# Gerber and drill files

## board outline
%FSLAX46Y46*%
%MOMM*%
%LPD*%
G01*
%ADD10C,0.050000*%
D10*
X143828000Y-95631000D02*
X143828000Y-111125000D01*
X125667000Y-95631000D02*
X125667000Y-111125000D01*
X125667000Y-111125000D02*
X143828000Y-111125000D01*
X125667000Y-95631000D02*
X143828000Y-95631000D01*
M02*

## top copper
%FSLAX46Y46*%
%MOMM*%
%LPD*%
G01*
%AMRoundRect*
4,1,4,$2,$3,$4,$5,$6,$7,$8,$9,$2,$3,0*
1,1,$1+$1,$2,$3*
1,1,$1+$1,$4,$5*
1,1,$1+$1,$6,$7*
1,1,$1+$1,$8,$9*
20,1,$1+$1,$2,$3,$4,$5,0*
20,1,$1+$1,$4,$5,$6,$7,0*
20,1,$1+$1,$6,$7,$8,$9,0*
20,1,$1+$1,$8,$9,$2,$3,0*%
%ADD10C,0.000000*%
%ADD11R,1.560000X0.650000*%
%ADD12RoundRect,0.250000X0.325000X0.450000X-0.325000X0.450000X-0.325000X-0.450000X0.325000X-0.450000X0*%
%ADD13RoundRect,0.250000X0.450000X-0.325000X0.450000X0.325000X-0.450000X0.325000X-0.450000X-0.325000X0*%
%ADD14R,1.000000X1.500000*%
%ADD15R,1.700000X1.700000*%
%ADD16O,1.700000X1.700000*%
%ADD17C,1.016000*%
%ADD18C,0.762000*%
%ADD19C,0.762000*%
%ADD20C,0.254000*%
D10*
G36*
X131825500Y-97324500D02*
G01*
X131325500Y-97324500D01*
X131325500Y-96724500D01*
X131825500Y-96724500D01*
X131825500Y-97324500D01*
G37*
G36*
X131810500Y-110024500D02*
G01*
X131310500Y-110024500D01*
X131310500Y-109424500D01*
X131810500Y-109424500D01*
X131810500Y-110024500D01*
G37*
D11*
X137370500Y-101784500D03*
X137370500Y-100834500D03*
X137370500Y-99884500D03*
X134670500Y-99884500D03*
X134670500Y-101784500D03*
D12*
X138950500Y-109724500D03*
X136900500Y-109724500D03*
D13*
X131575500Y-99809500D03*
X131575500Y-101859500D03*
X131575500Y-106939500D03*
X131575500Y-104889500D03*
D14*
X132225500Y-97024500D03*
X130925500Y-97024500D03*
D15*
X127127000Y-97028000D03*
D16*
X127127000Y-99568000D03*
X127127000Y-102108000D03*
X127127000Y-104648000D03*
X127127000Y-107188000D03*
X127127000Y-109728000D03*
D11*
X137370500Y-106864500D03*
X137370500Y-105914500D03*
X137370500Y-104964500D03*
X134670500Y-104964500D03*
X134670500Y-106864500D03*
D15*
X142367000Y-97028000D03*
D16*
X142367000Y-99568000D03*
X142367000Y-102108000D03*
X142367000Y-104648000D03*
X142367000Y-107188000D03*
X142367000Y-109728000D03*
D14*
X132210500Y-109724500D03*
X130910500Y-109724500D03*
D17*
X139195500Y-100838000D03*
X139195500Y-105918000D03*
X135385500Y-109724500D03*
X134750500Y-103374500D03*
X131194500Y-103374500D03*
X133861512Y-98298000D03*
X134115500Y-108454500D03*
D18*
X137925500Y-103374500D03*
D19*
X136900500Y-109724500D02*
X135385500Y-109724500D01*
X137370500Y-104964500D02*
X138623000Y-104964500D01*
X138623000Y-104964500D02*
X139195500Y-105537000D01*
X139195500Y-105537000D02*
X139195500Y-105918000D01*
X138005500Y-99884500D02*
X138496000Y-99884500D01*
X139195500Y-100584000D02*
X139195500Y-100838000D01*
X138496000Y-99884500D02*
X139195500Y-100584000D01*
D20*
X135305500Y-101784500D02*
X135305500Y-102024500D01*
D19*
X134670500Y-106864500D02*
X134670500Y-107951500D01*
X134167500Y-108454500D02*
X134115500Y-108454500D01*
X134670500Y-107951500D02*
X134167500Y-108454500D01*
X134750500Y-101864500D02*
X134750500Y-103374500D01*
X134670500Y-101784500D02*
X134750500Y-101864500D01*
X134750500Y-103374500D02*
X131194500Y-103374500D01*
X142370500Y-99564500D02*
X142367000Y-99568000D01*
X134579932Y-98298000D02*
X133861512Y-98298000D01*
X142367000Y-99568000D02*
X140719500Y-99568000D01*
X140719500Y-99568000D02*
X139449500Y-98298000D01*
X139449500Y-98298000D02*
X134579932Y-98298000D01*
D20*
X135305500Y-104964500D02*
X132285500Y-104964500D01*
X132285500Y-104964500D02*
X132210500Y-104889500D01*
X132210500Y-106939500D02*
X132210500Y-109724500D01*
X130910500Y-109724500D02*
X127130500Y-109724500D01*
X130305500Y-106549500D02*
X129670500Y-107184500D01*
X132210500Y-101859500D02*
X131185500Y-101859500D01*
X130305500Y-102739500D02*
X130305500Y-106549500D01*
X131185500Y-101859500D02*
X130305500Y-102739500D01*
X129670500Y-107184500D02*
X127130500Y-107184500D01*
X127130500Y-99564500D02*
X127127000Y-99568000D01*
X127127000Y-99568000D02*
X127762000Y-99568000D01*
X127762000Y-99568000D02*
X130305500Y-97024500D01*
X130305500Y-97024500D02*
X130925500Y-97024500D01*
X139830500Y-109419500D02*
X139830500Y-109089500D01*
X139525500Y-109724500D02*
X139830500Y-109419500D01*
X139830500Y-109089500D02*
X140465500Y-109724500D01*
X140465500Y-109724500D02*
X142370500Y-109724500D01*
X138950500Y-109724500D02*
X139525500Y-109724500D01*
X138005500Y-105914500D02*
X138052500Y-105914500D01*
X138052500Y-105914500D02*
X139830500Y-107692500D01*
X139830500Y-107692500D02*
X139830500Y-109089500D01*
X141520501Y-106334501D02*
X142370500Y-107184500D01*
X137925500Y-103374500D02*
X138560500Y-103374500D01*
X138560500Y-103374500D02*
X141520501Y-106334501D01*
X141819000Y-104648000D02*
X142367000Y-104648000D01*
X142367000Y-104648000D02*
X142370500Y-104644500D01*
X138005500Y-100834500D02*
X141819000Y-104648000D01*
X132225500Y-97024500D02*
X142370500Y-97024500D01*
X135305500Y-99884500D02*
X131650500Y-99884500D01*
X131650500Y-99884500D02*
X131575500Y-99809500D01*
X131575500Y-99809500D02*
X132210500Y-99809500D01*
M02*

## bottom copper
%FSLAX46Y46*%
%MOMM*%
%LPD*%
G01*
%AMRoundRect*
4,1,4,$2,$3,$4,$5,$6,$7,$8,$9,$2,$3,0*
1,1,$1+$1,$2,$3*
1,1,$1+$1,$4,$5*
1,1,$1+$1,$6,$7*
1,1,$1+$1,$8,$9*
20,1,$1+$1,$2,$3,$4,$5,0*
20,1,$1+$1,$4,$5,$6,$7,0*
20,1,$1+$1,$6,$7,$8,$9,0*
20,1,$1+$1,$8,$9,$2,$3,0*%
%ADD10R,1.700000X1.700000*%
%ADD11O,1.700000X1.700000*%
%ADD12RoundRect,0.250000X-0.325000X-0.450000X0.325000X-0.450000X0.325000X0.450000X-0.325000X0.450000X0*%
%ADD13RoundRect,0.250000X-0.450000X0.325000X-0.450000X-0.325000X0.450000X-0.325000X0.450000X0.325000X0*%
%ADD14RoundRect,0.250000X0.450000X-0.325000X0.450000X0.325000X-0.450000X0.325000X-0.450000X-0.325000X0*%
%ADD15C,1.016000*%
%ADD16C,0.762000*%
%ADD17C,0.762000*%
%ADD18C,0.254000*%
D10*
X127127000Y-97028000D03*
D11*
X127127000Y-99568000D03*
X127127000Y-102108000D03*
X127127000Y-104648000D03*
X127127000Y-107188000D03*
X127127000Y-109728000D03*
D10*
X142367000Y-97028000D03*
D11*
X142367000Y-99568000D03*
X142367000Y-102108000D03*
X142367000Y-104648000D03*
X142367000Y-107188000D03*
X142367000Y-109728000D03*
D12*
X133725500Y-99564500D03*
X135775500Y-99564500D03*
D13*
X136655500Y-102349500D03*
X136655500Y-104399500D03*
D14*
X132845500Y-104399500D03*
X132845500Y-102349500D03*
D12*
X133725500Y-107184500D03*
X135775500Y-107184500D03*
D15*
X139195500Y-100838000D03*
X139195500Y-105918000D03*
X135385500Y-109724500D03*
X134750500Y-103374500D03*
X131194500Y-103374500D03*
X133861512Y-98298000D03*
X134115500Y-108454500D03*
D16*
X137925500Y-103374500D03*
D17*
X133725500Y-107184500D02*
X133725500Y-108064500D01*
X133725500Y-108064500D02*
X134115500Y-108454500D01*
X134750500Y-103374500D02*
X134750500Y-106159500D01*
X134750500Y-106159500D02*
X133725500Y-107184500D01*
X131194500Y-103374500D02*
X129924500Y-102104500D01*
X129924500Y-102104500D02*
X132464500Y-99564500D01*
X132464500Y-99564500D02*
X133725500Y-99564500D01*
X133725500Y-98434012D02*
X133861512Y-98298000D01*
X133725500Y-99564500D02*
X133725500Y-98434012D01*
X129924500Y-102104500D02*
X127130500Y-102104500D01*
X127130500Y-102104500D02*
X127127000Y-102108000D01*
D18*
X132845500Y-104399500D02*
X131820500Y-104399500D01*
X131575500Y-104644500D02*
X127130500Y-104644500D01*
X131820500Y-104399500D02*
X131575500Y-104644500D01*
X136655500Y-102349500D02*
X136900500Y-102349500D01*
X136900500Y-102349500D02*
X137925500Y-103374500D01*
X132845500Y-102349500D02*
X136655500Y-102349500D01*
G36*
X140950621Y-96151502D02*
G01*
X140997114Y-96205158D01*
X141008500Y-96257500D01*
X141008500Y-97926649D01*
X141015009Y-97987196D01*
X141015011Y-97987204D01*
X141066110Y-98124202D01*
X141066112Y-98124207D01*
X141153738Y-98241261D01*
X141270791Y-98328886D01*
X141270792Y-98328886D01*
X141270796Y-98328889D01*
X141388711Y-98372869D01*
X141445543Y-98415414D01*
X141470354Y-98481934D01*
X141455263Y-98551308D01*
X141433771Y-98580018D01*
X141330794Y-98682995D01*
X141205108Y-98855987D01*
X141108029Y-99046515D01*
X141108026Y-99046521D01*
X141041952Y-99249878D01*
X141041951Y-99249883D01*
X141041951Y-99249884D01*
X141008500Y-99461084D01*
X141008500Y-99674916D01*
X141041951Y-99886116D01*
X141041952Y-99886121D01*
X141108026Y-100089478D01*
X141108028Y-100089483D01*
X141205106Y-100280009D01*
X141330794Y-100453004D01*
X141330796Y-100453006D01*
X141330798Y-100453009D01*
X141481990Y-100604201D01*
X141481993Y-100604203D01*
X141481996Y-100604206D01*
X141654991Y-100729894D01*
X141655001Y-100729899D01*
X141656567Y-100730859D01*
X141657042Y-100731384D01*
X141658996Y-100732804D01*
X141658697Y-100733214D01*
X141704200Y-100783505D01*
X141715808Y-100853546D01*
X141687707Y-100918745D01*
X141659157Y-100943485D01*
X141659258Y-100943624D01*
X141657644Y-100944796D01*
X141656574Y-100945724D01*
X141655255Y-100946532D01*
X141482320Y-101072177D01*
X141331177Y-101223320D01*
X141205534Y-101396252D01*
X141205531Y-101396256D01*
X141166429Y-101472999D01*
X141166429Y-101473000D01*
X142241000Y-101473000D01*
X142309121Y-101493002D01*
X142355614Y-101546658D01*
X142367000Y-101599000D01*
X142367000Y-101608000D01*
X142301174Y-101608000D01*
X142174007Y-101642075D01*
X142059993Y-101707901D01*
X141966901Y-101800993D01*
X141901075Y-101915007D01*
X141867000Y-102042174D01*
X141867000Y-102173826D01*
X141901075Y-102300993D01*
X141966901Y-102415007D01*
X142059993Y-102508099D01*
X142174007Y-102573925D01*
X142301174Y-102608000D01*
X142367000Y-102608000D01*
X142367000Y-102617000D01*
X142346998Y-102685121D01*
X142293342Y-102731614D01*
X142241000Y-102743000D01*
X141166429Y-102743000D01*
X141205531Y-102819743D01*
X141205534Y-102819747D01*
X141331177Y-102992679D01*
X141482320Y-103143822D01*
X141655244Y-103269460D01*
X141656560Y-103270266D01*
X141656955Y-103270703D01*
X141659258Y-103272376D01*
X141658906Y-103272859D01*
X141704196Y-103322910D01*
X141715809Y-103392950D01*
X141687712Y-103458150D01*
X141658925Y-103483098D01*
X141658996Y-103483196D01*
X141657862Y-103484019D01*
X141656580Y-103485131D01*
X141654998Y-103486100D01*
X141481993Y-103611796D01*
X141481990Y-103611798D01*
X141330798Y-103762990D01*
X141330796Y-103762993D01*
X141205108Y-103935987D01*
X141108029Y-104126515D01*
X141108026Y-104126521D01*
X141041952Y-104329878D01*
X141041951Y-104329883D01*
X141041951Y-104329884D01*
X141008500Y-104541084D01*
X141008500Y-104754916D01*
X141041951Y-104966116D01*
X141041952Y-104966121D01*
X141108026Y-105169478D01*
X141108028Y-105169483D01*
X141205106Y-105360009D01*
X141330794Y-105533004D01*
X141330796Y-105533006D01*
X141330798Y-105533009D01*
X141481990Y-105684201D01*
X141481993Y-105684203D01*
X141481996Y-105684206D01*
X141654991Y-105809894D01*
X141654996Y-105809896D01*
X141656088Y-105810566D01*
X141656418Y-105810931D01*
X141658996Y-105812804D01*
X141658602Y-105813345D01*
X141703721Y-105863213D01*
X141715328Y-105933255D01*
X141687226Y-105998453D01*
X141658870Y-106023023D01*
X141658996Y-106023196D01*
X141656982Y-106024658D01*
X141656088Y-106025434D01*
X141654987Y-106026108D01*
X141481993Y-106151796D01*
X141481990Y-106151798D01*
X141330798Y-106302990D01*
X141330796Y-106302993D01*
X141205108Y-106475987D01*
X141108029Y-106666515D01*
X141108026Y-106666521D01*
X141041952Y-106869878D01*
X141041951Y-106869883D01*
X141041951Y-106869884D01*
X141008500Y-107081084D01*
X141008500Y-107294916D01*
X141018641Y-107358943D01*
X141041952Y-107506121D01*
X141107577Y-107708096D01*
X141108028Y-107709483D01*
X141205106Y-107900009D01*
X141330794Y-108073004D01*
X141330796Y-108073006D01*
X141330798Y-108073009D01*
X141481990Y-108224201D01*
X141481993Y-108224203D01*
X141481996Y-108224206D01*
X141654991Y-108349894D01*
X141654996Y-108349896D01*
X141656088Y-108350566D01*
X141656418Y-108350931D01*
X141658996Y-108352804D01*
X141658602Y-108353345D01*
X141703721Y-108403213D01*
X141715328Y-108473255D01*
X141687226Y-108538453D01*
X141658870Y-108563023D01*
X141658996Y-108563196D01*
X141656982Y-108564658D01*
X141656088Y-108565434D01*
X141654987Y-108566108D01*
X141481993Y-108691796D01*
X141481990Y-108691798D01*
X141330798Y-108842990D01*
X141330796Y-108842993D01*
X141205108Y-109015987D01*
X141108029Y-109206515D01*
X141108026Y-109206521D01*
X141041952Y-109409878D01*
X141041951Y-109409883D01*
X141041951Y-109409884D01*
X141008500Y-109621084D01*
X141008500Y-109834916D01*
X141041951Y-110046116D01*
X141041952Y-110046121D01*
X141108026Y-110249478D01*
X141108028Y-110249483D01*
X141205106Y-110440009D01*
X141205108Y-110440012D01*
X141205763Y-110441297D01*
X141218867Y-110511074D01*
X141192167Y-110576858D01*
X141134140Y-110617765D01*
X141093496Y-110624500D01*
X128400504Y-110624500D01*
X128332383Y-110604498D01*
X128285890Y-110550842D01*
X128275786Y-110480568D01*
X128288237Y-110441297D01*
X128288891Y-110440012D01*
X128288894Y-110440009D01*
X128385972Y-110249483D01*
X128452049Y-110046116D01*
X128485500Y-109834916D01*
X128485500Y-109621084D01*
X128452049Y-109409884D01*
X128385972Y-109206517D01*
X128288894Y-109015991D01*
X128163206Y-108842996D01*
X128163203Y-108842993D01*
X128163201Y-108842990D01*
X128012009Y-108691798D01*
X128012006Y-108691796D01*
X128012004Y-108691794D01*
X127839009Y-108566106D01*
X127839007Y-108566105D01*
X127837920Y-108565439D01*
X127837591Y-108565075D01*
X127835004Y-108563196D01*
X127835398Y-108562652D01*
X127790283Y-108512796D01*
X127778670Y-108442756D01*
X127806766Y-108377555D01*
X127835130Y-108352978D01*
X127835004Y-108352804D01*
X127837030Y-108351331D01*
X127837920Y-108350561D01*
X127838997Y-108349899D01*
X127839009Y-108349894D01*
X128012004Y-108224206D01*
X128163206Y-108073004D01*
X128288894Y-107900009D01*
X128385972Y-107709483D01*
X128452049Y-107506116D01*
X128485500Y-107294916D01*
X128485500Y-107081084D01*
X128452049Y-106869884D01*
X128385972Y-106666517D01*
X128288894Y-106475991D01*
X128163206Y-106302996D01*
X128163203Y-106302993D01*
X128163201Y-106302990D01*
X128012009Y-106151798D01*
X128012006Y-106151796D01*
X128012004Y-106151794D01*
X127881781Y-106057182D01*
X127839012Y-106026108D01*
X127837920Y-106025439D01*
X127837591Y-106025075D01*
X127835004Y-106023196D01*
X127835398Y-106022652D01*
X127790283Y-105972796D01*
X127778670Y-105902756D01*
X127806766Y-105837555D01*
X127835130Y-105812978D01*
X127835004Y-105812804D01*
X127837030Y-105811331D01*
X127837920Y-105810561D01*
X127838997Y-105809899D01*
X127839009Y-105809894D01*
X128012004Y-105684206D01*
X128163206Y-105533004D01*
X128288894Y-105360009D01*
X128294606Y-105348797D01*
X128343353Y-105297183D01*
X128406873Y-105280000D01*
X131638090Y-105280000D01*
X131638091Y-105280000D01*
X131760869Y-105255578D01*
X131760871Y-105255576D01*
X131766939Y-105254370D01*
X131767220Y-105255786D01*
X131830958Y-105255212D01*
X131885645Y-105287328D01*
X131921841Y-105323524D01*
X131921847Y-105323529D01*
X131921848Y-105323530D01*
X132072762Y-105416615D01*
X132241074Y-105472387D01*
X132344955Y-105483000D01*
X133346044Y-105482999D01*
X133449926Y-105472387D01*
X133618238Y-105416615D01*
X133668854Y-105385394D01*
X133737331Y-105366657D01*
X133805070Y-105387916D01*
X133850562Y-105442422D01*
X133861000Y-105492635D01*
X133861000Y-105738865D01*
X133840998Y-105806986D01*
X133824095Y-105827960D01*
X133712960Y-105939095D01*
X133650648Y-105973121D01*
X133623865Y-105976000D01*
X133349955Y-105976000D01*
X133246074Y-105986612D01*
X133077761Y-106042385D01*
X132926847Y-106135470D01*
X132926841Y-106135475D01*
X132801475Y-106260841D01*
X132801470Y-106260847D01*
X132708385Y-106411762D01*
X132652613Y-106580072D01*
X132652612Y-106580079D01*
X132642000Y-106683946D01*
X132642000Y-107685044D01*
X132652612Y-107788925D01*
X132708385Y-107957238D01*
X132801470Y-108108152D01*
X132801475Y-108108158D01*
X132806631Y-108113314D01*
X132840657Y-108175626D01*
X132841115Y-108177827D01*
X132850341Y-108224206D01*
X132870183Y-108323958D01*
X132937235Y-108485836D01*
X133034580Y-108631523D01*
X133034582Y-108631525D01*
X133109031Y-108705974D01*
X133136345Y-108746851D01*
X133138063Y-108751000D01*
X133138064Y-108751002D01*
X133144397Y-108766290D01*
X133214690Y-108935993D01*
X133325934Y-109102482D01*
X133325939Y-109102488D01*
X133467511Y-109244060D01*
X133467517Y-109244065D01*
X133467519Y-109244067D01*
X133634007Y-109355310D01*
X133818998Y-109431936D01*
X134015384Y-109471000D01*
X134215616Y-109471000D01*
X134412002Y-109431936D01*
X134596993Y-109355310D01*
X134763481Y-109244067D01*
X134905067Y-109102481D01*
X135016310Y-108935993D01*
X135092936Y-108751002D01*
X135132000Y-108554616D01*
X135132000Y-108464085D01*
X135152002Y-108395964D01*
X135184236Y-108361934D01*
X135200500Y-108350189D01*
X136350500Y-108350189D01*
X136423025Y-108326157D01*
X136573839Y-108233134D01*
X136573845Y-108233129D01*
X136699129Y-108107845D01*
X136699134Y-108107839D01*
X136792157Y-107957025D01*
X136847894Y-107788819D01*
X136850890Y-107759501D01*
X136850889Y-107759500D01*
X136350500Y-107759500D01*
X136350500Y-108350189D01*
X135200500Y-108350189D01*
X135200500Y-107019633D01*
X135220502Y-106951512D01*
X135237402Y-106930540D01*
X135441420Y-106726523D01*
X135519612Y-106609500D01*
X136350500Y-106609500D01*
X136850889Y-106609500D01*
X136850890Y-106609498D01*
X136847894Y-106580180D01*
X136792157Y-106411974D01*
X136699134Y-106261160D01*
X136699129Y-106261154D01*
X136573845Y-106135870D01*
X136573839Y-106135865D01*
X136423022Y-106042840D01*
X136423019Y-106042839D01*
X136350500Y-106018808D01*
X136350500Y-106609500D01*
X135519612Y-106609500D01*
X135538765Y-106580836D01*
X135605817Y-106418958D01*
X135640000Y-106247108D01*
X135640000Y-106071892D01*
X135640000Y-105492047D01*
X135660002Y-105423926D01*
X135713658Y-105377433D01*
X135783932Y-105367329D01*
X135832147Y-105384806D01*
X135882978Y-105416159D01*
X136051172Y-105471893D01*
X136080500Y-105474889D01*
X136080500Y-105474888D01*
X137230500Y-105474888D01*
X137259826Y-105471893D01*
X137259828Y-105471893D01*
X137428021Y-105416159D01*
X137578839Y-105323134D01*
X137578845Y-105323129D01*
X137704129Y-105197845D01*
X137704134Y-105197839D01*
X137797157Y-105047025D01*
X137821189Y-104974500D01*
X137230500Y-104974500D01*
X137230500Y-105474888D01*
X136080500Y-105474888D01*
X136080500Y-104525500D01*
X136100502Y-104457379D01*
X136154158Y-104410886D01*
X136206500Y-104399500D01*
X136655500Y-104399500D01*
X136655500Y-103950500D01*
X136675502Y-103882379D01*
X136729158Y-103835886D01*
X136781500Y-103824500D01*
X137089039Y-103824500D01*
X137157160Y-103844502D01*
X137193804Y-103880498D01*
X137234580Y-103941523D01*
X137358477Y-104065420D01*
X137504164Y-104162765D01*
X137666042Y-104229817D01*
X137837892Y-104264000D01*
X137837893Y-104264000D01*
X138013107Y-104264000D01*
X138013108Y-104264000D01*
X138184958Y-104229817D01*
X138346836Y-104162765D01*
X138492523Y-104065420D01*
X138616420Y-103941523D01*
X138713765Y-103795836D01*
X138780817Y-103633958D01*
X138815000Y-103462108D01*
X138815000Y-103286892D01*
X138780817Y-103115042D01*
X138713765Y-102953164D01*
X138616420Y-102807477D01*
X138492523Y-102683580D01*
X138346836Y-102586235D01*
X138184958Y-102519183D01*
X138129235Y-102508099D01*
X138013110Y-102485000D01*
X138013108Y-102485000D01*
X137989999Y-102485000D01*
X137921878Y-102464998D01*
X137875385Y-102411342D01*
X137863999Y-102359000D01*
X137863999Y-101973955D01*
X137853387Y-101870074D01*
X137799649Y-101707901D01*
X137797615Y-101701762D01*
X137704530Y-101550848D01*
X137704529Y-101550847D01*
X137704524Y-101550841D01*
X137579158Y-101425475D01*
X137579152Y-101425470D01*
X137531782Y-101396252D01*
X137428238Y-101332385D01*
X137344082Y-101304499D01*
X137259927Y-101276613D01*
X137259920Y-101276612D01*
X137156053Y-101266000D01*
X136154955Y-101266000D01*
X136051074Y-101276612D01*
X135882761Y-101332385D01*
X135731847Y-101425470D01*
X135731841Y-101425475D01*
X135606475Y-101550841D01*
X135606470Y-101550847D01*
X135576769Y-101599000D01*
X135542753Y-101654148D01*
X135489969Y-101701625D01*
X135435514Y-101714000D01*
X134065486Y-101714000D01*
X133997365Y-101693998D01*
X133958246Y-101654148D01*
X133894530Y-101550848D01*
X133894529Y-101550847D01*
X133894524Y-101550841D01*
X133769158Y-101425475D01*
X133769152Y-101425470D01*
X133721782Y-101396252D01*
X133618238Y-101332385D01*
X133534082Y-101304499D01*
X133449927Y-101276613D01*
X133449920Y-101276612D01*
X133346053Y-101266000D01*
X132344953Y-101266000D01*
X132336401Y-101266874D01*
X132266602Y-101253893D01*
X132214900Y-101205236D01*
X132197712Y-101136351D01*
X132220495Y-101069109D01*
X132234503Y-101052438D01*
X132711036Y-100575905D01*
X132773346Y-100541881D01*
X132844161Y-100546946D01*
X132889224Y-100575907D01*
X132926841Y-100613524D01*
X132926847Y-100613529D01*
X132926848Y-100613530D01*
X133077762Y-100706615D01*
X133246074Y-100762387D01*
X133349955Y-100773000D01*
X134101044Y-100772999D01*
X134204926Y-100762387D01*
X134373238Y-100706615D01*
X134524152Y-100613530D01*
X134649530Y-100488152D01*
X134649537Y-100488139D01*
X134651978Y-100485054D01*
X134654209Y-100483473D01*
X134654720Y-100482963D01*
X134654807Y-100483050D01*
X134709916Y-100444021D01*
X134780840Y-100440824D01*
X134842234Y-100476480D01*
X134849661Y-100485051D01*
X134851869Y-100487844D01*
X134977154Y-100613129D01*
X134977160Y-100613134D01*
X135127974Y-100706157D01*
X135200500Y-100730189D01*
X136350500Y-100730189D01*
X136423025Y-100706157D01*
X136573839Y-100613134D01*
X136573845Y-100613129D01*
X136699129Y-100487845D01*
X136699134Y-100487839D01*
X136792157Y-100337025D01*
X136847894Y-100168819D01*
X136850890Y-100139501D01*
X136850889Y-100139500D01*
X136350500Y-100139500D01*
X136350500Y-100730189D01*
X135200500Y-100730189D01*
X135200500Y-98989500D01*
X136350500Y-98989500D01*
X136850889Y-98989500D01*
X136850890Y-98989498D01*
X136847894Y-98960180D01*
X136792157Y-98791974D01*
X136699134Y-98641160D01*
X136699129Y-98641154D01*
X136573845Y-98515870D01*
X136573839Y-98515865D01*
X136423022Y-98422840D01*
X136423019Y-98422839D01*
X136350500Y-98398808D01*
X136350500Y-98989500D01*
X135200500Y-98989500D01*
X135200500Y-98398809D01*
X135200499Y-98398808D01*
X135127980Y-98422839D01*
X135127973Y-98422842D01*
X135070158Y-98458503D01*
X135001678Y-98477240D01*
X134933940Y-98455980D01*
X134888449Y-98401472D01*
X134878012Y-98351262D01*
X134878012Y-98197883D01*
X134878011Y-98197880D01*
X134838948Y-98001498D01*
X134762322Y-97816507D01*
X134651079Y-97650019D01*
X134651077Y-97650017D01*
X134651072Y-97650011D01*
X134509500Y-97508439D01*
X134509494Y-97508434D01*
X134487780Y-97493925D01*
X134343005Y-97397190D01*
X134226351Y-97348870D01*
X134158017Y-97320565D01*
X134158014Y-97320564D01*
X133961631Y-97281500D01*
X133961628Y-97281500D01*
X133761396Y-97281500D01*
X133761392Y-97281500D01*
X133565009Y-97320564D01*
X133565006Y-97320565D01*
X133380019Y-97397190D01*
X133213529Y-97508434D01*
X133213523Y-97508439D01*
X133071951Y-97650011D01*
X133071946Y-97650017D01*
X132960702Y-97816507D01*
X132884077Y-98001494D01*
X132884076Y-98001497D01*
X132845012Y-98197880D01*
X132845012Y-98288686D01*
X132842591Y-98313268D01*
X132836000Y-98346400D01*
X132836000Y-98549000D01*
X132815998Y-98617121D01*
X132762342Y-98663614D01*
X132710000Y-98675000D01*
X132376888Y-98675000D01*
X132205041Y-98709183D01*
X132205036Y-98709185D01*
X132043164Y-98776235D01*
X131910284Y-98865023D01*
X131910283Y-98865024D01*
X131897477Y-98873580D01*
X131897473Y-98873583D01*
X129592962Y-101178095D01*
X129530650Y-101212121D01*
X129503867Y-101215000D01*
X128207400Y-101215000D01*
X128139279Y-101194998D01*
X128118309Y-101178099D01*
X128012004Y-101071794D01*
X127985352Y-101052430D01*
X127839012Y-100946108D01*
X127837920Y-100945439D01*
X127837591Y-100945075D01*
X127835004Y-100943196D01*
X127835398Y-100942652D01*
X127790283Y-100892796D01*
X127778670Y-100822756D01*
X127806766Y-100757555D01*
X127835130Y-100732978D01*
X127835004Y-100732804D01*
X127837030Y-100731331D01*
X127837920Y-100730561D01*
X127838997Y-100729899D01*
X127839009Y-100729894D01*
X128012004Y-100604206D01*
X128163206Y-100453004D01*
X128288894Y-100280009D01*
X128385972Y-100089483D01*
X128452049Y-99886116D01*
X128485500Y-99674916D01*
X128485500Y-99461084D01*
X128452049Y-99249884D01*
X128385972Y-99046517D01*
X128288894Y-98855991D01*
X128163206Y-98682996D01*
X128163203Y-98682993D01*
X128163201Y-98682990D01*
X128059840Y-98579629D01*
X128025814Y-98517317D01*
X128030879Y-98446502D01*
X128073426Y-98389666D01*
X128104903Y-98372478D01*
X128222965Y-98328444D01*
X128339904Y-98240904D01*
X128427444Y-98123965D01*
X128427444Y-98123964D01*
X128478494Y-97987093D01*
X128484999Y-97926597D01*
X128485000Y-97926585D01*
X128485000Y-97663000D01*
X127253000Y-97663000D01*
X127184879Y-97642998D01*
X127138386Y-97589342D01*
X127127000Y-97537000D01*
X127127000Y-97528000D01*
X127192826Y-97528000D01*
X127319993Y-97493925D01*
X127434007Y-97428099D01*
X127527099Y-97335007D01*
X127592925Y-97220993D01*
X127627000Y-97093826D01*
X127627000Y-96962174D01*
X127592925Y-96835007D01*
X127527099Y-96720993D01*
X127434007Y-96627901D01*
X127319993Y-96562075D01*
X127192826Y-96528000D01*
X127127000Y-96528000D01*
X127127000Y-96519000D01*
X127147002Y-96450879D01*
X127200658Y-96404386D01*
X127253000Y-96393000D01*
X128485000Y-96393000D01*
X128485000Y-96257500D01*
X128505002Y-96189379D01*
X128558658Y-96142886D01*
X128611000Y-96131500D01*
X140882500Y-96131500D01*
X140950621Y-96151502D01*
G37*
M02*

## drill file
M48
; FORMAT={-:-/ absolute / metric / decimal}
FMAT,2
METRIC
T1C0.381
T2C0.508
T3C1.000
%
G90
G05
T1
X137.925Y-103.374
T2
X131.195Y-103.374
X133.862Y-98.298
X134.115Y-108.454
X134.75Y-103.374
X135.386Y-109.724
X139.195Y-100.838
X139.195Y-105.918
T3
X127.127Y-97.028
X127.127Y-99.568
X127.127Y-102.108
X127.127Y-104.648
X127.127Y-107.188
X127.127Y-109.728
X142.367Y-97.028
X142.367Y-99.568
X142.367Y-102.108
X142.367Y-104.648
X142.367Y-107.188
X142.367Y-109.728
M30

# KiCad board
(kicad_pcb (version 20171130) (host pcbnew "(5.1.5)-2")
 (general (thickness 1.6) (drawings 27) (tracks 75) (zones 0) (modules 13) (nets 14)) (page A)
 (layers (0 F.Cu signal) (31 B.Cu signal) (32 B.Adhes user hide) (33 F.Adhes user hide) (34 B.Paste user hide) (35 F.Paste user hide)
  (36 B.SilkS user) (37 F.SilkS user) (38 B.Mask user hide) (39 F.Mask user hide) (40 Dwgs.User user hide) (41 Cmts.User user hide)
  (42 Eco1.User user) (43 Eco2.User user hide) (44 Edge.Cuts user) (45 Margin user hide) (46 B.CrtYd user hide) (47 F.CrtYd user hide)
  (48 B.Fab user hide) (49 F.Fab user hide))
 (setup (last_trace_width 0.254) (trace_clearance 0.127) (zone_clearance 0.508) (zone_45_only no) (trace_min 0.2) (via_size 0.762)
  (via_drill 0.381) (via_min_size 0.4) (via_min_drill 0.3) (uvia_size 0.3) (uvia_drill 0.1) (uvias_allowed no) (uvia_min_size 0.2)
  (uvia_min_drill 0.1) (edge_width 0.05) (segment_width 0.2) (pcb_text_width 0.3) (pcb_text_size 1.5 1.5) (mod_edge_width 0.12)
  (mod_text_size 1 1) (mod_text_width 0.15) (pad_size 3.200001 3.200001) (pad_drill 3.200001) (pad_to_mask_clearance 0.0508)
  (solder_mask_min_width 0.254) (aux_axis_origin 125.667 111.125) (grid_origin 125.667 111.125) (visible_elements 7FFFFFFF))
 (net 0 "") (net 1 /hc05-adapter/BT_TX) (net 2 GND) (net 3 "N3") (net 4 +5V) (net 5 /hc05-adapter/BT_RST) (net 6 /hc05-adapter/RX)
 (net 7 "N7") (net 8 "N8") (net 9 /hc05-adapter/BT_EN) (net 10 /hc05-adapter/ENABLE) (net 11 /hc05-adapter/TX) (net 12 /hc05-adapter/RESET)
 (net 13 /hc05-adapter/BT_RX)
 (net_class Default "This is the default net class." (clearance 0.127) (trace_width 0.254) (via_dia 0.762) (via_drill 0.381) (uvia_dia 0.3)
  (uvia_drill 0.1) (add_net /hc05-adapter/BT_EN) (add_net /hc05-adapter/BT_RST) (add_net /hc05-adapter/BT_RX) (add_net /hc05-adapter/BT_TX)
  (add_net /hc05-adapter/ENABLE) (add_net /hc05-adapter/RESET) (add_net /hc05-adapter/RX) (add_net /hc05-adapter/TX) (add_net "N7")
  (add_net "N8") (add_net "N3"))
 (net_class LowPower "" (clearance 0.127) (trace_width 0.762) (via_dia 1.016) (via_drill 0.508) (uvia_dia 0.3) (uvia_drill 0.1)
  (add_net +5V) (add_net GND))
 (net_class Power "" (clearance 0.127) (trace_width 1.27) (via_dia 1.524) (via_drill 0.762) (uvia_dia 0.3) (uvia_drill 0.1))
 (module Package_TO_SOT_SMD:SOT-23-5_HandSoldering (layer F.Cu) (at 136.0205 100.8345 180)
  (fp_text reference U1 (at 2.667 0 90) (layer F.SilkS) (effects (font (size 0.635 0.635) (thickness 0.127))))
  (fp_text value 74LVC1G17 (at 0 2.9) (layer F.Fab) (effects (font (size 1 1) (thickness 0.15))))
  (pad 1 smd rect (at -1.35 -0.95 180) (size 1.56 0.65) (layers F.Cu F.Paste F.Mask))
  (pad 2 smd rect (at -1.35 0 180) (size 1.56 0.65) (layers F.Cu F.Paste F.Mask) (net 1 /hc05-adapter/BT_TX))
  (pad 3 smd rect (at -1.35 0.95 180) (size 1.56 0.65) (layers F.Cu F.Paste F.Mask) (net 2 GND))
  (pad 4 smd rect (at 1.35 0.95 180) (size 1.56 0.65) (layers F.Cu F.Paste F.Mask) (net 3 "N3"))
  (pad 5 smd rect (at 1.35 -0.95 180) (size 1.56 0.65) (layers F.Cu F.Paste F.Mask) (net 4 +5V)))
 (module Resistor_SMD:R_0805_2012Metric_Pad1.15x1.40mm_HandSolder (layer F.Cu) (at 137.9255 109.7245 180)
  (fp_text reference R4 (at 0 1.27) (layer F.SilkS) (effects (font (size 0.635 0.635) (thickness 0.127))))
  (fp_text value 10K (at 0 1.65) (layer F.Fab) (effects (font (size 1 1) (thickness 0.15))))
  (pad 1 smd roundrect (at -1.025 0 180) (size 1.15 1.4) (layers F.Cu F.Paste F.Mask) (roundrect_rratio 0.217391)
   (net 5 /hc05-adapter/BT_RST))
  (pad 2 smd roundrect (at 1.025 0 180) (size 1.15 1.4) (layers F.Cu F.Paste F.Mask) (roundrect_rratio 0.217391) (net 2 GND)))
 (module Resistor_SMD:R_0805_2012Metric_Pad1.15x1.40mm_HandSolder (layer F.Cu) (at 131.5755 100.8345 90)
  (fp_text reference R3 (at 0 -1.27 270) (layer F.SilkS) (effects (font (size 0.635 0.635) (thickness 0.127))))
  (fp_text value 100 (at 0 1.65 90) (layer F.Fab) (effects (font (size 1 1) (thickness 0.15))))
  (pad 2 smd roundrect (at 1.025 0 90) (size 1.15 1.4) (layers F.Cu F.Paste F.Mask) (roundrect_rratio 0.217391) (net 3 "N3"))
  (pad 1 smd roundrect (at -1.025 0 90) (size 1.15 1.4) (layers F.Cu F.Paste F.Mask) (roundrect_rratio 0.217391) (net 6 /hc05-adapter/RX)))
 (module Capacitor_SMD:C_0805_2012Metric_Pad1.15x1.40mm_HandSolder (layer F.Cu) (at 131.5755 105.9145 90)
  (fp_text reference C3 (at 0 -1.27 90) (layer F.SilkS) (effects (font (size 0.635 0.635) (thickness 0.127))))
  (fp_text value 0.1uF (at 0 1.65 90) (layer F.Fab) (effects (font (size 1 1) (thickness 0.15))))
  (pad 1 smd roundrect (at -1.025 0 90) (size 1.15 1.4) (layers F.Cu F.Paste F.Mask) (roundrect_rratio 0.217391) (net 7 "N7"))
  (pad 2 smd roundrect (at 1.025 0 90) (size 1.15 1.4) (layers F.Cu F.Paste F.Mask) (roundrect_rratio 0.217391) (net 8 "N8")))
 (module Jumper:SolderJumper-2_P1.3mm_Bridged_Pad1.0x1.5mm (layer F.Cu) (at 131.5755 97.0245 180)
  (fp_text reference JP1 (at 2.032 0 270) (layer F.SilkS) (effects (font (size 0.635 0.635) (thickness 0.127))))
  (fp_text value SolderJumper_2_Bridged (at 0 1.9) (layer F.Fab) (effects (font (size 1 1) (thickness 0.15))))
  (fp_poly (pts (xy -0.25 -0.3) (xy 0.25 -0.3) (xy 0.25 0.3) (xy -0.25 0.3)) (layer F.Cu) (width 0))
  (pad 1 smd rect (at -0.65 0 180) (size 1 1.5) (layers F.Cu F.Mask) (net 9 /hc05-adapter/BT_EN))
  (pad 2 smd rect (at 0.65 0 180) (size 1 1.5) (layers F.Cu F.Mask) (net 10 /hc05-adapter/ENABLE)))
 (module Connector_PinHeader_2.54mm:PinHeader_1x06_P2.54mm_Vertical (layer F.Cu) (at 127.127 97.028)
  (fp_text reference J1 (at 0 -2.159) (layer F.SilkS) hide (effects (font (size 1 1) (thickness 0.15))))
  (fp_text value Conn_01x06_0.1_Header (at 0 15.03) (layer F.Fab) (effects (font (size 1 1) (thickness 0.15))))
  (pad 1 thru_hole rect (at 0 0) (size 1.7 1.7) (drill 1) (layers *.Cu *.Mask) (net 2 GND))
  (pad 2 thru_hole oval (at 0 2.54) (size 1.7 1.7) (drill 1) (layers *.Cu *.Mask) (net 10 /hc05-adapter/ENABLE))
  (pad 3 thru_hole oval (at 0 5.08) (size 1.7 1.7) (drill 1) (layers *.Cu *.Mask) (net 4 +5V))
  (pad 4 thru_hole oval (at 0 7.62) (size 1.7 1.7) (drill 1) (layers *.Cu *.Mask) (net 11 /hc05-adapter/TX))
  (pad 5 thru_hole oval (at 0 10.16) (size 1.7 1.7) (drill 1) (layers *.Cu *.Mask) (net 6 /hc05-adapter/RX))
  (pad 6 thru_hole oval (at 0 12.7) (size 1.7 1.7) (drill 1) (layers *.Cu *.Mask) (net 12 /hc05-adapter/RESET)))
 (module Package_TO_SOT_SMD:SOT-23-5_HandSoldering (layer F.Cu) (at 136.0205 105.9145 180)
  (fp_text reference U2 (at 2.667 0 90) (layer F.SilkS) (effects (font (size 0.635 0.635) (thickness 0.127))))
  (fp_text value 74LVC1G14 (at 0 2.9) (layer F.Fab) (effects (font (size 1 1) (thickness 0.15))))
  (pad 1 smd rect (at -1.35 -0.95 180) (size 1.56 0.65) (layers F.Cu F.Paste F.Mask))
  (pad 2 smd rect (at -1.35 0 180) (size 1.56 0.65) (layers F.Cu F.Paste F.Mask) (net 5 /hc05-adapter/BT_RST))
  (pad 3 smd rect (at -1.35 0.95 180) (size 1.56 0.65) (layers F.Cu F.Paste F.Mask) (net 2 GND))
  (pad 4 smd rect (at 1.35 0.95 180) (size 1.56 0.65) (layers F.Cu F.Paste F.Mask) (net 8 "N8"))
  (pad 5 smd rect (at 1.35 -0.95 180) (size 1.56 0.65) (layers F.Cu F.Paste F.Mask) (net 4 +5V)))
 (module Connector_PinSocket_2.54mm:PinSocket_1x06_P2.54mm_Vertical (layer F.Cu) (at 142.367 97.028)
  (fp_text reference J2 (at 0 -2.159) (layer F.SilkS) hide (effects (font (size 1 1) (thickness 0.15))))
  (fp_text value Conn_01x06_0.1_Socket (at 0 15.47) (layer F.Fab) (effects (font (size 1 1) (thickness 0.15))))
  (pad 1 thru_hole rect (at 0 0) (size 1.7 1.7) (drill 1) (layers *.Cu *.Mask) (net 9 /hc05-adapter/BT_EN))
  (pad 2 thru_hole oval (at 0 2.54) (size 1.7 1.7) (drill 1) (layers *.Cu *.Mask) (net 4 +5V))
  (pad 3 thru_hole oval (at 0 5.08) (size 1.7 1.7) (drill 1) (layers *.Cu *.Mask) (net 2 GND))
  (pad 4 thru_hole oval (at 0 7.62) (size 1.7 1.7) (drill 1) (layers *.Cu *.Mask) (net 1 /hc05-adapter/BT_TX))
  (pad 5 thru_hole oval (at 0 10.16) (size 1.7 1.7) (drill 1) (layers *.Cu *.Mask) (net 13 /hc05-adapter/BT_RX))
  (pad 6 thru_hole oval (at 0 12.7) (size 1.7 1.7) (drill 1) (layers *.Cu *.Mask) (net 5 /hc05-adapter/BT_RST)))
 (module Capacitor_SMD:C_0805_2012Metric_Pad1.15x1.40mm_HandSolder (layer B.Cu) (at 134.7505 99.5645)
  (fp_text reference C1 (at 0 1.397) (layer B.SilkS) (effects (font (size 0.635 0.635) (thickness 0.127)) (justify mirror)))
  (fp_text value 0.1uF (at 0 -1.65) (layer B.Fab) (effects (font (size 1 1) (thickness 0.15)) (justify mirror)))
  (pad 1 smd roundrect (at -1.025 0) (size 1.15 1.4) (layers B.Cu B.Paste B.Mask) (roundrect_rratio 0.217391) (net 4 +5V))
  (pad 2 smd roundrect (at 1.025 0) (size 1.15 1.4) (layers B.Cu B.Paste B.Mask) (roundrect_rratio 0.217391) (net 2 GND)))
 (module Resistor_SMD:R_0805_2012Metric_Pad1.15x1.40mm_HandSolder (layer B.Cu) (at 136.6555 103.3745 270)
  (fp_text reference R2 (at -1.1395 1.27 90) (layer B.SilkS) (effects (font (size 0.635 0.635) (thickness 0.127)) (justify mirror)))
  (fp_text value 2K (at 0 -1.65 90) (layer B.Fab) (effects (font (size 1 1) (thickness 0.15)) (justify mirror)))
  (pad 1 smd roundrect (at -1.025 0 270) (size 1.15 1.4) (layers B.Cu B.Paste B.Mask) (roundrect_rratio 0.217391)
   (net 13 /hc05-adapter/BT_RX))
  (pad 2 smd roundrect (at 1.025 0 270) (size 1.15 1.4) (layers B.Cu B.Paste B.Mask) (roundrect_rratio 0.217391) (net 2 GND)))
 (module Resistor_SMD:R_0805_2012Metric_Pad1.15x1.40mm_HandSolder (layer B.Cu) (at 132.8455 103.3745 90)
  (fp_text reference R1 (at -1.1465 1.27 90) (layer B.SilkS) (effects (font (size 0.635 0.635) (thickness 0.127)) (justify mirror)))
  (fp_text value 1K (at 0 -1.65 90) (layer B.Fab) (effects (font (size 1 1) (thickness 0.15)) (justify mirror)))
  (pad 1 smd roundrect (at -1.025 0 90) (size 1.15 1.4) (layers B.Cu B.Paste B.Mask) (roundrect_rratio 0.217391) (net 11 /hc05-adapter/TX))
  (pad 2 smd roundrect (at 1.025 0 90) (size 1.15 1.4) (layers B.Cu B.Paste B.Mask) (roundrect_rratio 0.217391) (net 13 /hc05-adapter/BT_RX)))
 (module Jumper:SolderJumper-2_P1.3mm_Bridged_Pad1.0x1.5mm (layer F.Cu) (at 131.5605 109.7245 180)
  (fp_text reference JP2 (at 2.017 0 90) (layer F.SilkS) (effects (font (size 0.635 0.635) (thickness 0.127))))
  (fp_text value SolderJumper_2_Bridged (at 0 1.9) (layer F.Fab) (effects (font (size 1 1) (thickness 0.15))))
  (fp_poly (pts (xy -0.25 -0.3) (xy 0.25 -0.3) (xy 0.25 0.3) (xy -0.25 0.3)) (layer F.Cu) (width 0))
  (pad 1 smd rect (at -0.65 0 180) (size 1 1.5) (layers F.Cu F.Mask) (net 7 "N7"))
  (pad 2 smd rect (at 0.65 0 180) (size 1 1.5) (layers F.Cu F.Mask) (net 12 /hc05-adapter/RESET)))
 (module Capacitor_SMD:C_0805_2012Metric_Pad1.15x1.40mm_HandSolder (layer B.Cu) (at 134.7505 107.1845)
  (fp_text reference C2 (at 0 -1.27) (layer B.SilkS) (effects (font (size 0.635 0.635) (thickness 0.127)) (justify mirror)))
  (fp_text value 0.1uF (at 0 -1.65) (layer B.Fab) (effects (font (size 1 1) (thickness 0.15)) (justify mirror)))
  (pad 1 smd roundrect (at -1.025 0) (size 1.15 1.4) (layers B.Cu B.Paste B.Mask) (roundrect_rratio 0.217391) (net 4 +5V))
  (pad 2 smd roundrect (at 1.025 0) (size 1.15 1.4) (layers B.Cu B.Paste B.Mask) (roundrect_rratio 0.217391) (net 2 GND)))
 (gr_line (start 143.828 95.631) (end 143.828 111.125) (layer Edge.Cuts) (width 0.05))
 (gr_line (start 125.667 95.631) (end 125.667 111.125) (layer Edge.Cuts) (width 0.05))
 (gr_line (start 125.667 111.125) (end 143.828 111.125) (layer Edge.Cuts) (width 0.05))
 (gr_line (start 125.667 95.631) (end 143.828 95.631) (layer Edge.Cuts) (width 0.05))
 (via (at 139.1955 100.838) (size 1.016) (drill 0.508) (layers F.Cu B.Cu) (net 2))
 (via (at 139.1955 105.918) (size 1.016) (drill 0.508) (layers F.Cu B.Cu) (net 2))
 (via (at 135.3855 109.7245) (size 1.016) (drill 0.508) (layers F.Cu B.Cu) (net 2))
 (segment (start 136.9005 109.7245) (end 135.3855 109.7245) (width 0.762) (layer F.Cu) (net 2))
 (segment (start 137.3705 104.9645) (end 138.623 104.9645) (width 0.762) (layer F.Cu) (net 2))
 (segment (start 138.623 104.9645) (end 139.1955 105.537) (width 0.762) (layer F.Cu) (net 2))
 (segment (start 139.1955 105.537) (end 139.1955 105.918) (width 0.762) (layer F.Cu) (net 2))
 (segment (start 138.0055 99.8845) (end 138.496 99.8845) (width 0.762) (layer F.Cu) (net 2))
 (segment (start 139.1955 100.584) (end 139.1955 100.838) (width 0.762) (layer F.Cu) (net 2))
 (segment (start 138.496 99.8845) (end 139.1955 100.584) (width 0.762) (layer F.Cu) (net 2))
 (via (at 134.7505 103.3745) (size 1.016) (drill 0.508) (layers F.Cu B.Cu) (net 4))
 (via (at 131.1945 103.3745) (size 1.016) (drill 0.508) (layers F.Cu B.Cu) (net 4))
 (segment (start 135.3055 101.7845) (end 135.3055 102.0245) (width 0.254) (layer F.Cu) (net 4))
 (segment (start 134.6705 106.8645) (end 134.6705 107.9515) (width 0.762) (layer F.Cu) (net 4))
 (segment (start 133.7255 107.1845) (end 133.7255 108.0645) (width 0.762) (layer B.Cu) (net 4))
 (segment (start 134.1675 108.4545) (end 134.1155 108.4545) (width 0.762) (layer F.Cu) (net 4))
 (segment (start 134.6705 107.9515) (end 134.1675 108.4545) (width 0.762) (layer F.Cu) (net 4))
 (segment (start 133.7255 108.0645) (end 134.1155 108.4545) (width 0.762) (layer B.Cu) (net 4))
 (via (at 133.861512 98.298) (size 1.016) (drill 0.508) (layers F.Cu B.Cu) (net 4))
 (segment (start 134.7505 101.8645) (end 134.7505 103.3745) (width 0.762) (layer F.Cu) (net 4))
 (segment (start 134.6705 101.7845) (end 134.7505 101.8645) (width 0.762) (layer F.Cu) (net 4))
 (segment (start 134.7505 103.3745) (end 134.7505 106.1595) (width 0.762) (layer B.Cu) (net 4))
 (segment (start 134.7505 106.1595) (end 133.7255 107.1845) (width 0.762) (layer B.Cu) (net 4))
 (segment (start 134.7505 103.3745) (end 131.1945 103.3745) (width 0.762) (layer F.Cu) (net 4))
 (segment (start 142.3705 99.5645) (end 142.367 99.568) (width 0.762) (layer F.Cu) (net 4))
 (segment (start 134.579932 98.298) (end 133.861512 98.298) (width 0.762) (layer F.Cu) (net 4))
 (segment (start 142.367 99.568) (end 140.7195 99.568) (width 0.762) (layer F.Cu) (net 4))
 (segment (start 140.7195 99.568) (end 139.4495 98.298) (width 0.762) (layer F.Cu) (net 4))
 (segment (start 139.4495 98.298) (end 134.579932 98.298) (width 0.762) (layer F.Cu) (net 4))
 (segment (start 131.1945 103.3745) (end 129.9245 102.1045) (width 0.762) (layer B.Cu) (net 4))
 (segment (start 129.9245 102.1045) (end 132.4645 99.5645) (width 0.762) (layer B.Cu) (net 4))
 (segment (start 132.4645 99.5645) (end 133.7255 99.5645) (width 0.762) (layer B.Cu) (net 4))
 (via (at 134.1155 108.4545) (size 1.016) (drill 0.508) (layers F.Cu B.Cu) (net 4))
 (segment (start 133.7255 98.434012) (end 133.861512 98.298) (width 0.762) (layer B.Cu) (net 4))
 (segment (start 133.7255 99.5645) (end 133.7255 98.434012) (width 0.762) (layer B.Cu) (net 4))
 (segment (start 129.9245 102.1045) (end 127.1305 102.1045) (width 0.762) (layer B.Cu) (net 4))
 (segment (start 127.1305 102.1045) (end 127.127 102.108) (width 0.762) (layer B.Cu) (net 4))
 (segment (start 135.3055 104.9645) (end 132.2855 104.9645) (width 0.254) (layer F.Cu) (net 8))
 (segment (start 132.2855 104.9645) (end 132.2105 104.8895) (width 0.254) (layer F.Cu) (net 8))
 (segment (start 132.2105 106.9395) (end 132.2105 109.7245) (width 0.254) (layer F.Cu) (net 7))
 (segment (start 130.9105 109.7245) (end 127.1305 109.7245) (width 0.254) (layer F.Cu) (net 12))
 (segment (start 130.3055 106.5495) (end 129.6705 107.1845) (width 0.254) (layer F.Cu) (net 6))
 (segment (start 132.2105 101.8595) (end 131.1855 101.8595) (width 0.254) (layer F.Cu) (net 6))
 (segment (start 130.3055 102.7395) (end 130.3055 106.5495) (width 0.254) (layer F.Cu) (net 6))
 (segment (start 131.1855 101.8595) (end 130.3055 102.7395) (width 0.254) (layer F.Cu) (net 6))
 (segment (start 129.6705 107.1845) (end 127.1305 107.1845) (width 0.254) (layer F.Cu) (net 6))
 (segment (start 132.8455 104.3995) (end 131.8205 104.3995) (width 0.254) (layer B.Cu) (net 11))
 (segment (start 131.5755 104.6445) (end 127.1305 104.6445) (width 0.254) (layer B.Cu) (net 11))
 (segment (start 131.8205 104.3995) (end 131.5755 104.6445) (width 0.254) (layer B.Cu) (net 11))
 (segment (start 127.1305 99.5645) (end 127.127 99.568) (width 0.254) (layer F.Cu) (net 10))
 (segment (start 127.127 99.568) (end 127.762 99.568) (width 0.254) (layer F.Cu) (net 10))
 (segment (start 127.762 99.568) (end 130.3055 97.0245) (width 0.254) (layer F.Cu) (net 10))
 (segment (start 130.3055 97.0245) (end 130.9255 97.0245) (width 0.254) (layer F.Cu) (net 10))
 (segment (start 139.8305 109.4195) (end 139.8305 109.0895) (width 0.254) (layer F.Cu) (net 5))
 (segment (start 139.5255 109.7245) (end 139.8305 109.4195) (width 0.254) (layer F.Cu) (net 5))
 (segment (start 139.8305 109.0895) (end 140.4655 109.7245) (width 0.254) (layer F.Cu) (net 5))
 (segment (start 140.4655 109.7245) (end 142.3705 109.7245) (width 0.254) (layer F.Cu) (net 5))
 (segment (start 138.9505 109.7245) (end 139.5255 109.7245) (width 0.254) (layer F.Cu) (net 5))
 (segment (start 138.0055 105.9145) (end 138.0525 105.9145) (width 0.254) (layer F.Cu) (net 5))
 (segment (start 138.0525 105.9145) (end 139.8305 107.6925) (width 0.254) (layer F.Cu) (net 5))
 (segment (start 139.8305 107.6925) (end 139.8305 109.0895) (width 0.254) (layer F.Cu) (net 5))
 (via (at 137.9255 103.3745) (size 0.762) (drill 0.381) (layers F.Cu B.Cu) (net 13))
 (segment (start 136.6555 102.3495) (end 136.9005 102.3495) (width 0.254) (layer B.Cu) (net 13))
 (segment (start 136.9005 102.3495) (end 137.9255 103.3745) (width 0.254) (layer B.Cu) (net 13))
 (segment (start 132.8455 102.3495) (end 136.6555 102.3495) (width 0.254) (layer B.Cu) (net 13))
 (segment (start 141.520501 106.334501) (end 142.3705 107.1845) (width 0.254) (layer F.Cu) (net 13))
 (segment (start 137.9255 103.3745) (end 138.5605 103.3745) (width 0.254) (layer F.Cu) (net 13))
 (segment (start 138.5605 103.3745) (end 141.520501 106.334501) (width 0.254) (layer F.Cu) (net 13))
 (segment (start 141.819 104.648) (end 142.367 104.648) (width 0.254) (layer F.Cu) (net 1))
 (segment (start 142.367 104.648) (end 142.3705 104.6445) (width 0.254) (layer F.Cu) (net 1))
 (segment (start 138.0055 100.8345) (end 141.819 104.648) (width 0.254) (layer F.Cu) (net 1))
 (segment (start 132.2255 97.0245) (end 142.3705 97.0245) (width 0.254) (layer F.Cu) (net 9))
 (segment (start 135.3055 99.8845) (end 131.6505 99.8845) (width 0.254) (layer F.Cu) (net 3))
 (segment (start 131.6505 99.8845) (end 131.5755 99.8095) (width 0.254) (layer F.Cu) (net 3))
 (segment (start 131.5755 99.8095) (end 132.2105 99.8095) (width 0.254) (layer F.Cu) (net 3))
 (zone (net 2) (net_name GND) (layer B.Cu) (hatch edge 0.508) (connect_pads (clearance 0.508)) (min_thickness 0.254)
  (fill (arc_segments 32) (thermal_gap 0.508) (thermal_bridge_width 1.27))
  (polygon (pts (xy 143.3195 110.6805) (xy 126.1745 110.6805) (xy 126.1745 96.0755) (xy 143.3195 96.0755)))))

